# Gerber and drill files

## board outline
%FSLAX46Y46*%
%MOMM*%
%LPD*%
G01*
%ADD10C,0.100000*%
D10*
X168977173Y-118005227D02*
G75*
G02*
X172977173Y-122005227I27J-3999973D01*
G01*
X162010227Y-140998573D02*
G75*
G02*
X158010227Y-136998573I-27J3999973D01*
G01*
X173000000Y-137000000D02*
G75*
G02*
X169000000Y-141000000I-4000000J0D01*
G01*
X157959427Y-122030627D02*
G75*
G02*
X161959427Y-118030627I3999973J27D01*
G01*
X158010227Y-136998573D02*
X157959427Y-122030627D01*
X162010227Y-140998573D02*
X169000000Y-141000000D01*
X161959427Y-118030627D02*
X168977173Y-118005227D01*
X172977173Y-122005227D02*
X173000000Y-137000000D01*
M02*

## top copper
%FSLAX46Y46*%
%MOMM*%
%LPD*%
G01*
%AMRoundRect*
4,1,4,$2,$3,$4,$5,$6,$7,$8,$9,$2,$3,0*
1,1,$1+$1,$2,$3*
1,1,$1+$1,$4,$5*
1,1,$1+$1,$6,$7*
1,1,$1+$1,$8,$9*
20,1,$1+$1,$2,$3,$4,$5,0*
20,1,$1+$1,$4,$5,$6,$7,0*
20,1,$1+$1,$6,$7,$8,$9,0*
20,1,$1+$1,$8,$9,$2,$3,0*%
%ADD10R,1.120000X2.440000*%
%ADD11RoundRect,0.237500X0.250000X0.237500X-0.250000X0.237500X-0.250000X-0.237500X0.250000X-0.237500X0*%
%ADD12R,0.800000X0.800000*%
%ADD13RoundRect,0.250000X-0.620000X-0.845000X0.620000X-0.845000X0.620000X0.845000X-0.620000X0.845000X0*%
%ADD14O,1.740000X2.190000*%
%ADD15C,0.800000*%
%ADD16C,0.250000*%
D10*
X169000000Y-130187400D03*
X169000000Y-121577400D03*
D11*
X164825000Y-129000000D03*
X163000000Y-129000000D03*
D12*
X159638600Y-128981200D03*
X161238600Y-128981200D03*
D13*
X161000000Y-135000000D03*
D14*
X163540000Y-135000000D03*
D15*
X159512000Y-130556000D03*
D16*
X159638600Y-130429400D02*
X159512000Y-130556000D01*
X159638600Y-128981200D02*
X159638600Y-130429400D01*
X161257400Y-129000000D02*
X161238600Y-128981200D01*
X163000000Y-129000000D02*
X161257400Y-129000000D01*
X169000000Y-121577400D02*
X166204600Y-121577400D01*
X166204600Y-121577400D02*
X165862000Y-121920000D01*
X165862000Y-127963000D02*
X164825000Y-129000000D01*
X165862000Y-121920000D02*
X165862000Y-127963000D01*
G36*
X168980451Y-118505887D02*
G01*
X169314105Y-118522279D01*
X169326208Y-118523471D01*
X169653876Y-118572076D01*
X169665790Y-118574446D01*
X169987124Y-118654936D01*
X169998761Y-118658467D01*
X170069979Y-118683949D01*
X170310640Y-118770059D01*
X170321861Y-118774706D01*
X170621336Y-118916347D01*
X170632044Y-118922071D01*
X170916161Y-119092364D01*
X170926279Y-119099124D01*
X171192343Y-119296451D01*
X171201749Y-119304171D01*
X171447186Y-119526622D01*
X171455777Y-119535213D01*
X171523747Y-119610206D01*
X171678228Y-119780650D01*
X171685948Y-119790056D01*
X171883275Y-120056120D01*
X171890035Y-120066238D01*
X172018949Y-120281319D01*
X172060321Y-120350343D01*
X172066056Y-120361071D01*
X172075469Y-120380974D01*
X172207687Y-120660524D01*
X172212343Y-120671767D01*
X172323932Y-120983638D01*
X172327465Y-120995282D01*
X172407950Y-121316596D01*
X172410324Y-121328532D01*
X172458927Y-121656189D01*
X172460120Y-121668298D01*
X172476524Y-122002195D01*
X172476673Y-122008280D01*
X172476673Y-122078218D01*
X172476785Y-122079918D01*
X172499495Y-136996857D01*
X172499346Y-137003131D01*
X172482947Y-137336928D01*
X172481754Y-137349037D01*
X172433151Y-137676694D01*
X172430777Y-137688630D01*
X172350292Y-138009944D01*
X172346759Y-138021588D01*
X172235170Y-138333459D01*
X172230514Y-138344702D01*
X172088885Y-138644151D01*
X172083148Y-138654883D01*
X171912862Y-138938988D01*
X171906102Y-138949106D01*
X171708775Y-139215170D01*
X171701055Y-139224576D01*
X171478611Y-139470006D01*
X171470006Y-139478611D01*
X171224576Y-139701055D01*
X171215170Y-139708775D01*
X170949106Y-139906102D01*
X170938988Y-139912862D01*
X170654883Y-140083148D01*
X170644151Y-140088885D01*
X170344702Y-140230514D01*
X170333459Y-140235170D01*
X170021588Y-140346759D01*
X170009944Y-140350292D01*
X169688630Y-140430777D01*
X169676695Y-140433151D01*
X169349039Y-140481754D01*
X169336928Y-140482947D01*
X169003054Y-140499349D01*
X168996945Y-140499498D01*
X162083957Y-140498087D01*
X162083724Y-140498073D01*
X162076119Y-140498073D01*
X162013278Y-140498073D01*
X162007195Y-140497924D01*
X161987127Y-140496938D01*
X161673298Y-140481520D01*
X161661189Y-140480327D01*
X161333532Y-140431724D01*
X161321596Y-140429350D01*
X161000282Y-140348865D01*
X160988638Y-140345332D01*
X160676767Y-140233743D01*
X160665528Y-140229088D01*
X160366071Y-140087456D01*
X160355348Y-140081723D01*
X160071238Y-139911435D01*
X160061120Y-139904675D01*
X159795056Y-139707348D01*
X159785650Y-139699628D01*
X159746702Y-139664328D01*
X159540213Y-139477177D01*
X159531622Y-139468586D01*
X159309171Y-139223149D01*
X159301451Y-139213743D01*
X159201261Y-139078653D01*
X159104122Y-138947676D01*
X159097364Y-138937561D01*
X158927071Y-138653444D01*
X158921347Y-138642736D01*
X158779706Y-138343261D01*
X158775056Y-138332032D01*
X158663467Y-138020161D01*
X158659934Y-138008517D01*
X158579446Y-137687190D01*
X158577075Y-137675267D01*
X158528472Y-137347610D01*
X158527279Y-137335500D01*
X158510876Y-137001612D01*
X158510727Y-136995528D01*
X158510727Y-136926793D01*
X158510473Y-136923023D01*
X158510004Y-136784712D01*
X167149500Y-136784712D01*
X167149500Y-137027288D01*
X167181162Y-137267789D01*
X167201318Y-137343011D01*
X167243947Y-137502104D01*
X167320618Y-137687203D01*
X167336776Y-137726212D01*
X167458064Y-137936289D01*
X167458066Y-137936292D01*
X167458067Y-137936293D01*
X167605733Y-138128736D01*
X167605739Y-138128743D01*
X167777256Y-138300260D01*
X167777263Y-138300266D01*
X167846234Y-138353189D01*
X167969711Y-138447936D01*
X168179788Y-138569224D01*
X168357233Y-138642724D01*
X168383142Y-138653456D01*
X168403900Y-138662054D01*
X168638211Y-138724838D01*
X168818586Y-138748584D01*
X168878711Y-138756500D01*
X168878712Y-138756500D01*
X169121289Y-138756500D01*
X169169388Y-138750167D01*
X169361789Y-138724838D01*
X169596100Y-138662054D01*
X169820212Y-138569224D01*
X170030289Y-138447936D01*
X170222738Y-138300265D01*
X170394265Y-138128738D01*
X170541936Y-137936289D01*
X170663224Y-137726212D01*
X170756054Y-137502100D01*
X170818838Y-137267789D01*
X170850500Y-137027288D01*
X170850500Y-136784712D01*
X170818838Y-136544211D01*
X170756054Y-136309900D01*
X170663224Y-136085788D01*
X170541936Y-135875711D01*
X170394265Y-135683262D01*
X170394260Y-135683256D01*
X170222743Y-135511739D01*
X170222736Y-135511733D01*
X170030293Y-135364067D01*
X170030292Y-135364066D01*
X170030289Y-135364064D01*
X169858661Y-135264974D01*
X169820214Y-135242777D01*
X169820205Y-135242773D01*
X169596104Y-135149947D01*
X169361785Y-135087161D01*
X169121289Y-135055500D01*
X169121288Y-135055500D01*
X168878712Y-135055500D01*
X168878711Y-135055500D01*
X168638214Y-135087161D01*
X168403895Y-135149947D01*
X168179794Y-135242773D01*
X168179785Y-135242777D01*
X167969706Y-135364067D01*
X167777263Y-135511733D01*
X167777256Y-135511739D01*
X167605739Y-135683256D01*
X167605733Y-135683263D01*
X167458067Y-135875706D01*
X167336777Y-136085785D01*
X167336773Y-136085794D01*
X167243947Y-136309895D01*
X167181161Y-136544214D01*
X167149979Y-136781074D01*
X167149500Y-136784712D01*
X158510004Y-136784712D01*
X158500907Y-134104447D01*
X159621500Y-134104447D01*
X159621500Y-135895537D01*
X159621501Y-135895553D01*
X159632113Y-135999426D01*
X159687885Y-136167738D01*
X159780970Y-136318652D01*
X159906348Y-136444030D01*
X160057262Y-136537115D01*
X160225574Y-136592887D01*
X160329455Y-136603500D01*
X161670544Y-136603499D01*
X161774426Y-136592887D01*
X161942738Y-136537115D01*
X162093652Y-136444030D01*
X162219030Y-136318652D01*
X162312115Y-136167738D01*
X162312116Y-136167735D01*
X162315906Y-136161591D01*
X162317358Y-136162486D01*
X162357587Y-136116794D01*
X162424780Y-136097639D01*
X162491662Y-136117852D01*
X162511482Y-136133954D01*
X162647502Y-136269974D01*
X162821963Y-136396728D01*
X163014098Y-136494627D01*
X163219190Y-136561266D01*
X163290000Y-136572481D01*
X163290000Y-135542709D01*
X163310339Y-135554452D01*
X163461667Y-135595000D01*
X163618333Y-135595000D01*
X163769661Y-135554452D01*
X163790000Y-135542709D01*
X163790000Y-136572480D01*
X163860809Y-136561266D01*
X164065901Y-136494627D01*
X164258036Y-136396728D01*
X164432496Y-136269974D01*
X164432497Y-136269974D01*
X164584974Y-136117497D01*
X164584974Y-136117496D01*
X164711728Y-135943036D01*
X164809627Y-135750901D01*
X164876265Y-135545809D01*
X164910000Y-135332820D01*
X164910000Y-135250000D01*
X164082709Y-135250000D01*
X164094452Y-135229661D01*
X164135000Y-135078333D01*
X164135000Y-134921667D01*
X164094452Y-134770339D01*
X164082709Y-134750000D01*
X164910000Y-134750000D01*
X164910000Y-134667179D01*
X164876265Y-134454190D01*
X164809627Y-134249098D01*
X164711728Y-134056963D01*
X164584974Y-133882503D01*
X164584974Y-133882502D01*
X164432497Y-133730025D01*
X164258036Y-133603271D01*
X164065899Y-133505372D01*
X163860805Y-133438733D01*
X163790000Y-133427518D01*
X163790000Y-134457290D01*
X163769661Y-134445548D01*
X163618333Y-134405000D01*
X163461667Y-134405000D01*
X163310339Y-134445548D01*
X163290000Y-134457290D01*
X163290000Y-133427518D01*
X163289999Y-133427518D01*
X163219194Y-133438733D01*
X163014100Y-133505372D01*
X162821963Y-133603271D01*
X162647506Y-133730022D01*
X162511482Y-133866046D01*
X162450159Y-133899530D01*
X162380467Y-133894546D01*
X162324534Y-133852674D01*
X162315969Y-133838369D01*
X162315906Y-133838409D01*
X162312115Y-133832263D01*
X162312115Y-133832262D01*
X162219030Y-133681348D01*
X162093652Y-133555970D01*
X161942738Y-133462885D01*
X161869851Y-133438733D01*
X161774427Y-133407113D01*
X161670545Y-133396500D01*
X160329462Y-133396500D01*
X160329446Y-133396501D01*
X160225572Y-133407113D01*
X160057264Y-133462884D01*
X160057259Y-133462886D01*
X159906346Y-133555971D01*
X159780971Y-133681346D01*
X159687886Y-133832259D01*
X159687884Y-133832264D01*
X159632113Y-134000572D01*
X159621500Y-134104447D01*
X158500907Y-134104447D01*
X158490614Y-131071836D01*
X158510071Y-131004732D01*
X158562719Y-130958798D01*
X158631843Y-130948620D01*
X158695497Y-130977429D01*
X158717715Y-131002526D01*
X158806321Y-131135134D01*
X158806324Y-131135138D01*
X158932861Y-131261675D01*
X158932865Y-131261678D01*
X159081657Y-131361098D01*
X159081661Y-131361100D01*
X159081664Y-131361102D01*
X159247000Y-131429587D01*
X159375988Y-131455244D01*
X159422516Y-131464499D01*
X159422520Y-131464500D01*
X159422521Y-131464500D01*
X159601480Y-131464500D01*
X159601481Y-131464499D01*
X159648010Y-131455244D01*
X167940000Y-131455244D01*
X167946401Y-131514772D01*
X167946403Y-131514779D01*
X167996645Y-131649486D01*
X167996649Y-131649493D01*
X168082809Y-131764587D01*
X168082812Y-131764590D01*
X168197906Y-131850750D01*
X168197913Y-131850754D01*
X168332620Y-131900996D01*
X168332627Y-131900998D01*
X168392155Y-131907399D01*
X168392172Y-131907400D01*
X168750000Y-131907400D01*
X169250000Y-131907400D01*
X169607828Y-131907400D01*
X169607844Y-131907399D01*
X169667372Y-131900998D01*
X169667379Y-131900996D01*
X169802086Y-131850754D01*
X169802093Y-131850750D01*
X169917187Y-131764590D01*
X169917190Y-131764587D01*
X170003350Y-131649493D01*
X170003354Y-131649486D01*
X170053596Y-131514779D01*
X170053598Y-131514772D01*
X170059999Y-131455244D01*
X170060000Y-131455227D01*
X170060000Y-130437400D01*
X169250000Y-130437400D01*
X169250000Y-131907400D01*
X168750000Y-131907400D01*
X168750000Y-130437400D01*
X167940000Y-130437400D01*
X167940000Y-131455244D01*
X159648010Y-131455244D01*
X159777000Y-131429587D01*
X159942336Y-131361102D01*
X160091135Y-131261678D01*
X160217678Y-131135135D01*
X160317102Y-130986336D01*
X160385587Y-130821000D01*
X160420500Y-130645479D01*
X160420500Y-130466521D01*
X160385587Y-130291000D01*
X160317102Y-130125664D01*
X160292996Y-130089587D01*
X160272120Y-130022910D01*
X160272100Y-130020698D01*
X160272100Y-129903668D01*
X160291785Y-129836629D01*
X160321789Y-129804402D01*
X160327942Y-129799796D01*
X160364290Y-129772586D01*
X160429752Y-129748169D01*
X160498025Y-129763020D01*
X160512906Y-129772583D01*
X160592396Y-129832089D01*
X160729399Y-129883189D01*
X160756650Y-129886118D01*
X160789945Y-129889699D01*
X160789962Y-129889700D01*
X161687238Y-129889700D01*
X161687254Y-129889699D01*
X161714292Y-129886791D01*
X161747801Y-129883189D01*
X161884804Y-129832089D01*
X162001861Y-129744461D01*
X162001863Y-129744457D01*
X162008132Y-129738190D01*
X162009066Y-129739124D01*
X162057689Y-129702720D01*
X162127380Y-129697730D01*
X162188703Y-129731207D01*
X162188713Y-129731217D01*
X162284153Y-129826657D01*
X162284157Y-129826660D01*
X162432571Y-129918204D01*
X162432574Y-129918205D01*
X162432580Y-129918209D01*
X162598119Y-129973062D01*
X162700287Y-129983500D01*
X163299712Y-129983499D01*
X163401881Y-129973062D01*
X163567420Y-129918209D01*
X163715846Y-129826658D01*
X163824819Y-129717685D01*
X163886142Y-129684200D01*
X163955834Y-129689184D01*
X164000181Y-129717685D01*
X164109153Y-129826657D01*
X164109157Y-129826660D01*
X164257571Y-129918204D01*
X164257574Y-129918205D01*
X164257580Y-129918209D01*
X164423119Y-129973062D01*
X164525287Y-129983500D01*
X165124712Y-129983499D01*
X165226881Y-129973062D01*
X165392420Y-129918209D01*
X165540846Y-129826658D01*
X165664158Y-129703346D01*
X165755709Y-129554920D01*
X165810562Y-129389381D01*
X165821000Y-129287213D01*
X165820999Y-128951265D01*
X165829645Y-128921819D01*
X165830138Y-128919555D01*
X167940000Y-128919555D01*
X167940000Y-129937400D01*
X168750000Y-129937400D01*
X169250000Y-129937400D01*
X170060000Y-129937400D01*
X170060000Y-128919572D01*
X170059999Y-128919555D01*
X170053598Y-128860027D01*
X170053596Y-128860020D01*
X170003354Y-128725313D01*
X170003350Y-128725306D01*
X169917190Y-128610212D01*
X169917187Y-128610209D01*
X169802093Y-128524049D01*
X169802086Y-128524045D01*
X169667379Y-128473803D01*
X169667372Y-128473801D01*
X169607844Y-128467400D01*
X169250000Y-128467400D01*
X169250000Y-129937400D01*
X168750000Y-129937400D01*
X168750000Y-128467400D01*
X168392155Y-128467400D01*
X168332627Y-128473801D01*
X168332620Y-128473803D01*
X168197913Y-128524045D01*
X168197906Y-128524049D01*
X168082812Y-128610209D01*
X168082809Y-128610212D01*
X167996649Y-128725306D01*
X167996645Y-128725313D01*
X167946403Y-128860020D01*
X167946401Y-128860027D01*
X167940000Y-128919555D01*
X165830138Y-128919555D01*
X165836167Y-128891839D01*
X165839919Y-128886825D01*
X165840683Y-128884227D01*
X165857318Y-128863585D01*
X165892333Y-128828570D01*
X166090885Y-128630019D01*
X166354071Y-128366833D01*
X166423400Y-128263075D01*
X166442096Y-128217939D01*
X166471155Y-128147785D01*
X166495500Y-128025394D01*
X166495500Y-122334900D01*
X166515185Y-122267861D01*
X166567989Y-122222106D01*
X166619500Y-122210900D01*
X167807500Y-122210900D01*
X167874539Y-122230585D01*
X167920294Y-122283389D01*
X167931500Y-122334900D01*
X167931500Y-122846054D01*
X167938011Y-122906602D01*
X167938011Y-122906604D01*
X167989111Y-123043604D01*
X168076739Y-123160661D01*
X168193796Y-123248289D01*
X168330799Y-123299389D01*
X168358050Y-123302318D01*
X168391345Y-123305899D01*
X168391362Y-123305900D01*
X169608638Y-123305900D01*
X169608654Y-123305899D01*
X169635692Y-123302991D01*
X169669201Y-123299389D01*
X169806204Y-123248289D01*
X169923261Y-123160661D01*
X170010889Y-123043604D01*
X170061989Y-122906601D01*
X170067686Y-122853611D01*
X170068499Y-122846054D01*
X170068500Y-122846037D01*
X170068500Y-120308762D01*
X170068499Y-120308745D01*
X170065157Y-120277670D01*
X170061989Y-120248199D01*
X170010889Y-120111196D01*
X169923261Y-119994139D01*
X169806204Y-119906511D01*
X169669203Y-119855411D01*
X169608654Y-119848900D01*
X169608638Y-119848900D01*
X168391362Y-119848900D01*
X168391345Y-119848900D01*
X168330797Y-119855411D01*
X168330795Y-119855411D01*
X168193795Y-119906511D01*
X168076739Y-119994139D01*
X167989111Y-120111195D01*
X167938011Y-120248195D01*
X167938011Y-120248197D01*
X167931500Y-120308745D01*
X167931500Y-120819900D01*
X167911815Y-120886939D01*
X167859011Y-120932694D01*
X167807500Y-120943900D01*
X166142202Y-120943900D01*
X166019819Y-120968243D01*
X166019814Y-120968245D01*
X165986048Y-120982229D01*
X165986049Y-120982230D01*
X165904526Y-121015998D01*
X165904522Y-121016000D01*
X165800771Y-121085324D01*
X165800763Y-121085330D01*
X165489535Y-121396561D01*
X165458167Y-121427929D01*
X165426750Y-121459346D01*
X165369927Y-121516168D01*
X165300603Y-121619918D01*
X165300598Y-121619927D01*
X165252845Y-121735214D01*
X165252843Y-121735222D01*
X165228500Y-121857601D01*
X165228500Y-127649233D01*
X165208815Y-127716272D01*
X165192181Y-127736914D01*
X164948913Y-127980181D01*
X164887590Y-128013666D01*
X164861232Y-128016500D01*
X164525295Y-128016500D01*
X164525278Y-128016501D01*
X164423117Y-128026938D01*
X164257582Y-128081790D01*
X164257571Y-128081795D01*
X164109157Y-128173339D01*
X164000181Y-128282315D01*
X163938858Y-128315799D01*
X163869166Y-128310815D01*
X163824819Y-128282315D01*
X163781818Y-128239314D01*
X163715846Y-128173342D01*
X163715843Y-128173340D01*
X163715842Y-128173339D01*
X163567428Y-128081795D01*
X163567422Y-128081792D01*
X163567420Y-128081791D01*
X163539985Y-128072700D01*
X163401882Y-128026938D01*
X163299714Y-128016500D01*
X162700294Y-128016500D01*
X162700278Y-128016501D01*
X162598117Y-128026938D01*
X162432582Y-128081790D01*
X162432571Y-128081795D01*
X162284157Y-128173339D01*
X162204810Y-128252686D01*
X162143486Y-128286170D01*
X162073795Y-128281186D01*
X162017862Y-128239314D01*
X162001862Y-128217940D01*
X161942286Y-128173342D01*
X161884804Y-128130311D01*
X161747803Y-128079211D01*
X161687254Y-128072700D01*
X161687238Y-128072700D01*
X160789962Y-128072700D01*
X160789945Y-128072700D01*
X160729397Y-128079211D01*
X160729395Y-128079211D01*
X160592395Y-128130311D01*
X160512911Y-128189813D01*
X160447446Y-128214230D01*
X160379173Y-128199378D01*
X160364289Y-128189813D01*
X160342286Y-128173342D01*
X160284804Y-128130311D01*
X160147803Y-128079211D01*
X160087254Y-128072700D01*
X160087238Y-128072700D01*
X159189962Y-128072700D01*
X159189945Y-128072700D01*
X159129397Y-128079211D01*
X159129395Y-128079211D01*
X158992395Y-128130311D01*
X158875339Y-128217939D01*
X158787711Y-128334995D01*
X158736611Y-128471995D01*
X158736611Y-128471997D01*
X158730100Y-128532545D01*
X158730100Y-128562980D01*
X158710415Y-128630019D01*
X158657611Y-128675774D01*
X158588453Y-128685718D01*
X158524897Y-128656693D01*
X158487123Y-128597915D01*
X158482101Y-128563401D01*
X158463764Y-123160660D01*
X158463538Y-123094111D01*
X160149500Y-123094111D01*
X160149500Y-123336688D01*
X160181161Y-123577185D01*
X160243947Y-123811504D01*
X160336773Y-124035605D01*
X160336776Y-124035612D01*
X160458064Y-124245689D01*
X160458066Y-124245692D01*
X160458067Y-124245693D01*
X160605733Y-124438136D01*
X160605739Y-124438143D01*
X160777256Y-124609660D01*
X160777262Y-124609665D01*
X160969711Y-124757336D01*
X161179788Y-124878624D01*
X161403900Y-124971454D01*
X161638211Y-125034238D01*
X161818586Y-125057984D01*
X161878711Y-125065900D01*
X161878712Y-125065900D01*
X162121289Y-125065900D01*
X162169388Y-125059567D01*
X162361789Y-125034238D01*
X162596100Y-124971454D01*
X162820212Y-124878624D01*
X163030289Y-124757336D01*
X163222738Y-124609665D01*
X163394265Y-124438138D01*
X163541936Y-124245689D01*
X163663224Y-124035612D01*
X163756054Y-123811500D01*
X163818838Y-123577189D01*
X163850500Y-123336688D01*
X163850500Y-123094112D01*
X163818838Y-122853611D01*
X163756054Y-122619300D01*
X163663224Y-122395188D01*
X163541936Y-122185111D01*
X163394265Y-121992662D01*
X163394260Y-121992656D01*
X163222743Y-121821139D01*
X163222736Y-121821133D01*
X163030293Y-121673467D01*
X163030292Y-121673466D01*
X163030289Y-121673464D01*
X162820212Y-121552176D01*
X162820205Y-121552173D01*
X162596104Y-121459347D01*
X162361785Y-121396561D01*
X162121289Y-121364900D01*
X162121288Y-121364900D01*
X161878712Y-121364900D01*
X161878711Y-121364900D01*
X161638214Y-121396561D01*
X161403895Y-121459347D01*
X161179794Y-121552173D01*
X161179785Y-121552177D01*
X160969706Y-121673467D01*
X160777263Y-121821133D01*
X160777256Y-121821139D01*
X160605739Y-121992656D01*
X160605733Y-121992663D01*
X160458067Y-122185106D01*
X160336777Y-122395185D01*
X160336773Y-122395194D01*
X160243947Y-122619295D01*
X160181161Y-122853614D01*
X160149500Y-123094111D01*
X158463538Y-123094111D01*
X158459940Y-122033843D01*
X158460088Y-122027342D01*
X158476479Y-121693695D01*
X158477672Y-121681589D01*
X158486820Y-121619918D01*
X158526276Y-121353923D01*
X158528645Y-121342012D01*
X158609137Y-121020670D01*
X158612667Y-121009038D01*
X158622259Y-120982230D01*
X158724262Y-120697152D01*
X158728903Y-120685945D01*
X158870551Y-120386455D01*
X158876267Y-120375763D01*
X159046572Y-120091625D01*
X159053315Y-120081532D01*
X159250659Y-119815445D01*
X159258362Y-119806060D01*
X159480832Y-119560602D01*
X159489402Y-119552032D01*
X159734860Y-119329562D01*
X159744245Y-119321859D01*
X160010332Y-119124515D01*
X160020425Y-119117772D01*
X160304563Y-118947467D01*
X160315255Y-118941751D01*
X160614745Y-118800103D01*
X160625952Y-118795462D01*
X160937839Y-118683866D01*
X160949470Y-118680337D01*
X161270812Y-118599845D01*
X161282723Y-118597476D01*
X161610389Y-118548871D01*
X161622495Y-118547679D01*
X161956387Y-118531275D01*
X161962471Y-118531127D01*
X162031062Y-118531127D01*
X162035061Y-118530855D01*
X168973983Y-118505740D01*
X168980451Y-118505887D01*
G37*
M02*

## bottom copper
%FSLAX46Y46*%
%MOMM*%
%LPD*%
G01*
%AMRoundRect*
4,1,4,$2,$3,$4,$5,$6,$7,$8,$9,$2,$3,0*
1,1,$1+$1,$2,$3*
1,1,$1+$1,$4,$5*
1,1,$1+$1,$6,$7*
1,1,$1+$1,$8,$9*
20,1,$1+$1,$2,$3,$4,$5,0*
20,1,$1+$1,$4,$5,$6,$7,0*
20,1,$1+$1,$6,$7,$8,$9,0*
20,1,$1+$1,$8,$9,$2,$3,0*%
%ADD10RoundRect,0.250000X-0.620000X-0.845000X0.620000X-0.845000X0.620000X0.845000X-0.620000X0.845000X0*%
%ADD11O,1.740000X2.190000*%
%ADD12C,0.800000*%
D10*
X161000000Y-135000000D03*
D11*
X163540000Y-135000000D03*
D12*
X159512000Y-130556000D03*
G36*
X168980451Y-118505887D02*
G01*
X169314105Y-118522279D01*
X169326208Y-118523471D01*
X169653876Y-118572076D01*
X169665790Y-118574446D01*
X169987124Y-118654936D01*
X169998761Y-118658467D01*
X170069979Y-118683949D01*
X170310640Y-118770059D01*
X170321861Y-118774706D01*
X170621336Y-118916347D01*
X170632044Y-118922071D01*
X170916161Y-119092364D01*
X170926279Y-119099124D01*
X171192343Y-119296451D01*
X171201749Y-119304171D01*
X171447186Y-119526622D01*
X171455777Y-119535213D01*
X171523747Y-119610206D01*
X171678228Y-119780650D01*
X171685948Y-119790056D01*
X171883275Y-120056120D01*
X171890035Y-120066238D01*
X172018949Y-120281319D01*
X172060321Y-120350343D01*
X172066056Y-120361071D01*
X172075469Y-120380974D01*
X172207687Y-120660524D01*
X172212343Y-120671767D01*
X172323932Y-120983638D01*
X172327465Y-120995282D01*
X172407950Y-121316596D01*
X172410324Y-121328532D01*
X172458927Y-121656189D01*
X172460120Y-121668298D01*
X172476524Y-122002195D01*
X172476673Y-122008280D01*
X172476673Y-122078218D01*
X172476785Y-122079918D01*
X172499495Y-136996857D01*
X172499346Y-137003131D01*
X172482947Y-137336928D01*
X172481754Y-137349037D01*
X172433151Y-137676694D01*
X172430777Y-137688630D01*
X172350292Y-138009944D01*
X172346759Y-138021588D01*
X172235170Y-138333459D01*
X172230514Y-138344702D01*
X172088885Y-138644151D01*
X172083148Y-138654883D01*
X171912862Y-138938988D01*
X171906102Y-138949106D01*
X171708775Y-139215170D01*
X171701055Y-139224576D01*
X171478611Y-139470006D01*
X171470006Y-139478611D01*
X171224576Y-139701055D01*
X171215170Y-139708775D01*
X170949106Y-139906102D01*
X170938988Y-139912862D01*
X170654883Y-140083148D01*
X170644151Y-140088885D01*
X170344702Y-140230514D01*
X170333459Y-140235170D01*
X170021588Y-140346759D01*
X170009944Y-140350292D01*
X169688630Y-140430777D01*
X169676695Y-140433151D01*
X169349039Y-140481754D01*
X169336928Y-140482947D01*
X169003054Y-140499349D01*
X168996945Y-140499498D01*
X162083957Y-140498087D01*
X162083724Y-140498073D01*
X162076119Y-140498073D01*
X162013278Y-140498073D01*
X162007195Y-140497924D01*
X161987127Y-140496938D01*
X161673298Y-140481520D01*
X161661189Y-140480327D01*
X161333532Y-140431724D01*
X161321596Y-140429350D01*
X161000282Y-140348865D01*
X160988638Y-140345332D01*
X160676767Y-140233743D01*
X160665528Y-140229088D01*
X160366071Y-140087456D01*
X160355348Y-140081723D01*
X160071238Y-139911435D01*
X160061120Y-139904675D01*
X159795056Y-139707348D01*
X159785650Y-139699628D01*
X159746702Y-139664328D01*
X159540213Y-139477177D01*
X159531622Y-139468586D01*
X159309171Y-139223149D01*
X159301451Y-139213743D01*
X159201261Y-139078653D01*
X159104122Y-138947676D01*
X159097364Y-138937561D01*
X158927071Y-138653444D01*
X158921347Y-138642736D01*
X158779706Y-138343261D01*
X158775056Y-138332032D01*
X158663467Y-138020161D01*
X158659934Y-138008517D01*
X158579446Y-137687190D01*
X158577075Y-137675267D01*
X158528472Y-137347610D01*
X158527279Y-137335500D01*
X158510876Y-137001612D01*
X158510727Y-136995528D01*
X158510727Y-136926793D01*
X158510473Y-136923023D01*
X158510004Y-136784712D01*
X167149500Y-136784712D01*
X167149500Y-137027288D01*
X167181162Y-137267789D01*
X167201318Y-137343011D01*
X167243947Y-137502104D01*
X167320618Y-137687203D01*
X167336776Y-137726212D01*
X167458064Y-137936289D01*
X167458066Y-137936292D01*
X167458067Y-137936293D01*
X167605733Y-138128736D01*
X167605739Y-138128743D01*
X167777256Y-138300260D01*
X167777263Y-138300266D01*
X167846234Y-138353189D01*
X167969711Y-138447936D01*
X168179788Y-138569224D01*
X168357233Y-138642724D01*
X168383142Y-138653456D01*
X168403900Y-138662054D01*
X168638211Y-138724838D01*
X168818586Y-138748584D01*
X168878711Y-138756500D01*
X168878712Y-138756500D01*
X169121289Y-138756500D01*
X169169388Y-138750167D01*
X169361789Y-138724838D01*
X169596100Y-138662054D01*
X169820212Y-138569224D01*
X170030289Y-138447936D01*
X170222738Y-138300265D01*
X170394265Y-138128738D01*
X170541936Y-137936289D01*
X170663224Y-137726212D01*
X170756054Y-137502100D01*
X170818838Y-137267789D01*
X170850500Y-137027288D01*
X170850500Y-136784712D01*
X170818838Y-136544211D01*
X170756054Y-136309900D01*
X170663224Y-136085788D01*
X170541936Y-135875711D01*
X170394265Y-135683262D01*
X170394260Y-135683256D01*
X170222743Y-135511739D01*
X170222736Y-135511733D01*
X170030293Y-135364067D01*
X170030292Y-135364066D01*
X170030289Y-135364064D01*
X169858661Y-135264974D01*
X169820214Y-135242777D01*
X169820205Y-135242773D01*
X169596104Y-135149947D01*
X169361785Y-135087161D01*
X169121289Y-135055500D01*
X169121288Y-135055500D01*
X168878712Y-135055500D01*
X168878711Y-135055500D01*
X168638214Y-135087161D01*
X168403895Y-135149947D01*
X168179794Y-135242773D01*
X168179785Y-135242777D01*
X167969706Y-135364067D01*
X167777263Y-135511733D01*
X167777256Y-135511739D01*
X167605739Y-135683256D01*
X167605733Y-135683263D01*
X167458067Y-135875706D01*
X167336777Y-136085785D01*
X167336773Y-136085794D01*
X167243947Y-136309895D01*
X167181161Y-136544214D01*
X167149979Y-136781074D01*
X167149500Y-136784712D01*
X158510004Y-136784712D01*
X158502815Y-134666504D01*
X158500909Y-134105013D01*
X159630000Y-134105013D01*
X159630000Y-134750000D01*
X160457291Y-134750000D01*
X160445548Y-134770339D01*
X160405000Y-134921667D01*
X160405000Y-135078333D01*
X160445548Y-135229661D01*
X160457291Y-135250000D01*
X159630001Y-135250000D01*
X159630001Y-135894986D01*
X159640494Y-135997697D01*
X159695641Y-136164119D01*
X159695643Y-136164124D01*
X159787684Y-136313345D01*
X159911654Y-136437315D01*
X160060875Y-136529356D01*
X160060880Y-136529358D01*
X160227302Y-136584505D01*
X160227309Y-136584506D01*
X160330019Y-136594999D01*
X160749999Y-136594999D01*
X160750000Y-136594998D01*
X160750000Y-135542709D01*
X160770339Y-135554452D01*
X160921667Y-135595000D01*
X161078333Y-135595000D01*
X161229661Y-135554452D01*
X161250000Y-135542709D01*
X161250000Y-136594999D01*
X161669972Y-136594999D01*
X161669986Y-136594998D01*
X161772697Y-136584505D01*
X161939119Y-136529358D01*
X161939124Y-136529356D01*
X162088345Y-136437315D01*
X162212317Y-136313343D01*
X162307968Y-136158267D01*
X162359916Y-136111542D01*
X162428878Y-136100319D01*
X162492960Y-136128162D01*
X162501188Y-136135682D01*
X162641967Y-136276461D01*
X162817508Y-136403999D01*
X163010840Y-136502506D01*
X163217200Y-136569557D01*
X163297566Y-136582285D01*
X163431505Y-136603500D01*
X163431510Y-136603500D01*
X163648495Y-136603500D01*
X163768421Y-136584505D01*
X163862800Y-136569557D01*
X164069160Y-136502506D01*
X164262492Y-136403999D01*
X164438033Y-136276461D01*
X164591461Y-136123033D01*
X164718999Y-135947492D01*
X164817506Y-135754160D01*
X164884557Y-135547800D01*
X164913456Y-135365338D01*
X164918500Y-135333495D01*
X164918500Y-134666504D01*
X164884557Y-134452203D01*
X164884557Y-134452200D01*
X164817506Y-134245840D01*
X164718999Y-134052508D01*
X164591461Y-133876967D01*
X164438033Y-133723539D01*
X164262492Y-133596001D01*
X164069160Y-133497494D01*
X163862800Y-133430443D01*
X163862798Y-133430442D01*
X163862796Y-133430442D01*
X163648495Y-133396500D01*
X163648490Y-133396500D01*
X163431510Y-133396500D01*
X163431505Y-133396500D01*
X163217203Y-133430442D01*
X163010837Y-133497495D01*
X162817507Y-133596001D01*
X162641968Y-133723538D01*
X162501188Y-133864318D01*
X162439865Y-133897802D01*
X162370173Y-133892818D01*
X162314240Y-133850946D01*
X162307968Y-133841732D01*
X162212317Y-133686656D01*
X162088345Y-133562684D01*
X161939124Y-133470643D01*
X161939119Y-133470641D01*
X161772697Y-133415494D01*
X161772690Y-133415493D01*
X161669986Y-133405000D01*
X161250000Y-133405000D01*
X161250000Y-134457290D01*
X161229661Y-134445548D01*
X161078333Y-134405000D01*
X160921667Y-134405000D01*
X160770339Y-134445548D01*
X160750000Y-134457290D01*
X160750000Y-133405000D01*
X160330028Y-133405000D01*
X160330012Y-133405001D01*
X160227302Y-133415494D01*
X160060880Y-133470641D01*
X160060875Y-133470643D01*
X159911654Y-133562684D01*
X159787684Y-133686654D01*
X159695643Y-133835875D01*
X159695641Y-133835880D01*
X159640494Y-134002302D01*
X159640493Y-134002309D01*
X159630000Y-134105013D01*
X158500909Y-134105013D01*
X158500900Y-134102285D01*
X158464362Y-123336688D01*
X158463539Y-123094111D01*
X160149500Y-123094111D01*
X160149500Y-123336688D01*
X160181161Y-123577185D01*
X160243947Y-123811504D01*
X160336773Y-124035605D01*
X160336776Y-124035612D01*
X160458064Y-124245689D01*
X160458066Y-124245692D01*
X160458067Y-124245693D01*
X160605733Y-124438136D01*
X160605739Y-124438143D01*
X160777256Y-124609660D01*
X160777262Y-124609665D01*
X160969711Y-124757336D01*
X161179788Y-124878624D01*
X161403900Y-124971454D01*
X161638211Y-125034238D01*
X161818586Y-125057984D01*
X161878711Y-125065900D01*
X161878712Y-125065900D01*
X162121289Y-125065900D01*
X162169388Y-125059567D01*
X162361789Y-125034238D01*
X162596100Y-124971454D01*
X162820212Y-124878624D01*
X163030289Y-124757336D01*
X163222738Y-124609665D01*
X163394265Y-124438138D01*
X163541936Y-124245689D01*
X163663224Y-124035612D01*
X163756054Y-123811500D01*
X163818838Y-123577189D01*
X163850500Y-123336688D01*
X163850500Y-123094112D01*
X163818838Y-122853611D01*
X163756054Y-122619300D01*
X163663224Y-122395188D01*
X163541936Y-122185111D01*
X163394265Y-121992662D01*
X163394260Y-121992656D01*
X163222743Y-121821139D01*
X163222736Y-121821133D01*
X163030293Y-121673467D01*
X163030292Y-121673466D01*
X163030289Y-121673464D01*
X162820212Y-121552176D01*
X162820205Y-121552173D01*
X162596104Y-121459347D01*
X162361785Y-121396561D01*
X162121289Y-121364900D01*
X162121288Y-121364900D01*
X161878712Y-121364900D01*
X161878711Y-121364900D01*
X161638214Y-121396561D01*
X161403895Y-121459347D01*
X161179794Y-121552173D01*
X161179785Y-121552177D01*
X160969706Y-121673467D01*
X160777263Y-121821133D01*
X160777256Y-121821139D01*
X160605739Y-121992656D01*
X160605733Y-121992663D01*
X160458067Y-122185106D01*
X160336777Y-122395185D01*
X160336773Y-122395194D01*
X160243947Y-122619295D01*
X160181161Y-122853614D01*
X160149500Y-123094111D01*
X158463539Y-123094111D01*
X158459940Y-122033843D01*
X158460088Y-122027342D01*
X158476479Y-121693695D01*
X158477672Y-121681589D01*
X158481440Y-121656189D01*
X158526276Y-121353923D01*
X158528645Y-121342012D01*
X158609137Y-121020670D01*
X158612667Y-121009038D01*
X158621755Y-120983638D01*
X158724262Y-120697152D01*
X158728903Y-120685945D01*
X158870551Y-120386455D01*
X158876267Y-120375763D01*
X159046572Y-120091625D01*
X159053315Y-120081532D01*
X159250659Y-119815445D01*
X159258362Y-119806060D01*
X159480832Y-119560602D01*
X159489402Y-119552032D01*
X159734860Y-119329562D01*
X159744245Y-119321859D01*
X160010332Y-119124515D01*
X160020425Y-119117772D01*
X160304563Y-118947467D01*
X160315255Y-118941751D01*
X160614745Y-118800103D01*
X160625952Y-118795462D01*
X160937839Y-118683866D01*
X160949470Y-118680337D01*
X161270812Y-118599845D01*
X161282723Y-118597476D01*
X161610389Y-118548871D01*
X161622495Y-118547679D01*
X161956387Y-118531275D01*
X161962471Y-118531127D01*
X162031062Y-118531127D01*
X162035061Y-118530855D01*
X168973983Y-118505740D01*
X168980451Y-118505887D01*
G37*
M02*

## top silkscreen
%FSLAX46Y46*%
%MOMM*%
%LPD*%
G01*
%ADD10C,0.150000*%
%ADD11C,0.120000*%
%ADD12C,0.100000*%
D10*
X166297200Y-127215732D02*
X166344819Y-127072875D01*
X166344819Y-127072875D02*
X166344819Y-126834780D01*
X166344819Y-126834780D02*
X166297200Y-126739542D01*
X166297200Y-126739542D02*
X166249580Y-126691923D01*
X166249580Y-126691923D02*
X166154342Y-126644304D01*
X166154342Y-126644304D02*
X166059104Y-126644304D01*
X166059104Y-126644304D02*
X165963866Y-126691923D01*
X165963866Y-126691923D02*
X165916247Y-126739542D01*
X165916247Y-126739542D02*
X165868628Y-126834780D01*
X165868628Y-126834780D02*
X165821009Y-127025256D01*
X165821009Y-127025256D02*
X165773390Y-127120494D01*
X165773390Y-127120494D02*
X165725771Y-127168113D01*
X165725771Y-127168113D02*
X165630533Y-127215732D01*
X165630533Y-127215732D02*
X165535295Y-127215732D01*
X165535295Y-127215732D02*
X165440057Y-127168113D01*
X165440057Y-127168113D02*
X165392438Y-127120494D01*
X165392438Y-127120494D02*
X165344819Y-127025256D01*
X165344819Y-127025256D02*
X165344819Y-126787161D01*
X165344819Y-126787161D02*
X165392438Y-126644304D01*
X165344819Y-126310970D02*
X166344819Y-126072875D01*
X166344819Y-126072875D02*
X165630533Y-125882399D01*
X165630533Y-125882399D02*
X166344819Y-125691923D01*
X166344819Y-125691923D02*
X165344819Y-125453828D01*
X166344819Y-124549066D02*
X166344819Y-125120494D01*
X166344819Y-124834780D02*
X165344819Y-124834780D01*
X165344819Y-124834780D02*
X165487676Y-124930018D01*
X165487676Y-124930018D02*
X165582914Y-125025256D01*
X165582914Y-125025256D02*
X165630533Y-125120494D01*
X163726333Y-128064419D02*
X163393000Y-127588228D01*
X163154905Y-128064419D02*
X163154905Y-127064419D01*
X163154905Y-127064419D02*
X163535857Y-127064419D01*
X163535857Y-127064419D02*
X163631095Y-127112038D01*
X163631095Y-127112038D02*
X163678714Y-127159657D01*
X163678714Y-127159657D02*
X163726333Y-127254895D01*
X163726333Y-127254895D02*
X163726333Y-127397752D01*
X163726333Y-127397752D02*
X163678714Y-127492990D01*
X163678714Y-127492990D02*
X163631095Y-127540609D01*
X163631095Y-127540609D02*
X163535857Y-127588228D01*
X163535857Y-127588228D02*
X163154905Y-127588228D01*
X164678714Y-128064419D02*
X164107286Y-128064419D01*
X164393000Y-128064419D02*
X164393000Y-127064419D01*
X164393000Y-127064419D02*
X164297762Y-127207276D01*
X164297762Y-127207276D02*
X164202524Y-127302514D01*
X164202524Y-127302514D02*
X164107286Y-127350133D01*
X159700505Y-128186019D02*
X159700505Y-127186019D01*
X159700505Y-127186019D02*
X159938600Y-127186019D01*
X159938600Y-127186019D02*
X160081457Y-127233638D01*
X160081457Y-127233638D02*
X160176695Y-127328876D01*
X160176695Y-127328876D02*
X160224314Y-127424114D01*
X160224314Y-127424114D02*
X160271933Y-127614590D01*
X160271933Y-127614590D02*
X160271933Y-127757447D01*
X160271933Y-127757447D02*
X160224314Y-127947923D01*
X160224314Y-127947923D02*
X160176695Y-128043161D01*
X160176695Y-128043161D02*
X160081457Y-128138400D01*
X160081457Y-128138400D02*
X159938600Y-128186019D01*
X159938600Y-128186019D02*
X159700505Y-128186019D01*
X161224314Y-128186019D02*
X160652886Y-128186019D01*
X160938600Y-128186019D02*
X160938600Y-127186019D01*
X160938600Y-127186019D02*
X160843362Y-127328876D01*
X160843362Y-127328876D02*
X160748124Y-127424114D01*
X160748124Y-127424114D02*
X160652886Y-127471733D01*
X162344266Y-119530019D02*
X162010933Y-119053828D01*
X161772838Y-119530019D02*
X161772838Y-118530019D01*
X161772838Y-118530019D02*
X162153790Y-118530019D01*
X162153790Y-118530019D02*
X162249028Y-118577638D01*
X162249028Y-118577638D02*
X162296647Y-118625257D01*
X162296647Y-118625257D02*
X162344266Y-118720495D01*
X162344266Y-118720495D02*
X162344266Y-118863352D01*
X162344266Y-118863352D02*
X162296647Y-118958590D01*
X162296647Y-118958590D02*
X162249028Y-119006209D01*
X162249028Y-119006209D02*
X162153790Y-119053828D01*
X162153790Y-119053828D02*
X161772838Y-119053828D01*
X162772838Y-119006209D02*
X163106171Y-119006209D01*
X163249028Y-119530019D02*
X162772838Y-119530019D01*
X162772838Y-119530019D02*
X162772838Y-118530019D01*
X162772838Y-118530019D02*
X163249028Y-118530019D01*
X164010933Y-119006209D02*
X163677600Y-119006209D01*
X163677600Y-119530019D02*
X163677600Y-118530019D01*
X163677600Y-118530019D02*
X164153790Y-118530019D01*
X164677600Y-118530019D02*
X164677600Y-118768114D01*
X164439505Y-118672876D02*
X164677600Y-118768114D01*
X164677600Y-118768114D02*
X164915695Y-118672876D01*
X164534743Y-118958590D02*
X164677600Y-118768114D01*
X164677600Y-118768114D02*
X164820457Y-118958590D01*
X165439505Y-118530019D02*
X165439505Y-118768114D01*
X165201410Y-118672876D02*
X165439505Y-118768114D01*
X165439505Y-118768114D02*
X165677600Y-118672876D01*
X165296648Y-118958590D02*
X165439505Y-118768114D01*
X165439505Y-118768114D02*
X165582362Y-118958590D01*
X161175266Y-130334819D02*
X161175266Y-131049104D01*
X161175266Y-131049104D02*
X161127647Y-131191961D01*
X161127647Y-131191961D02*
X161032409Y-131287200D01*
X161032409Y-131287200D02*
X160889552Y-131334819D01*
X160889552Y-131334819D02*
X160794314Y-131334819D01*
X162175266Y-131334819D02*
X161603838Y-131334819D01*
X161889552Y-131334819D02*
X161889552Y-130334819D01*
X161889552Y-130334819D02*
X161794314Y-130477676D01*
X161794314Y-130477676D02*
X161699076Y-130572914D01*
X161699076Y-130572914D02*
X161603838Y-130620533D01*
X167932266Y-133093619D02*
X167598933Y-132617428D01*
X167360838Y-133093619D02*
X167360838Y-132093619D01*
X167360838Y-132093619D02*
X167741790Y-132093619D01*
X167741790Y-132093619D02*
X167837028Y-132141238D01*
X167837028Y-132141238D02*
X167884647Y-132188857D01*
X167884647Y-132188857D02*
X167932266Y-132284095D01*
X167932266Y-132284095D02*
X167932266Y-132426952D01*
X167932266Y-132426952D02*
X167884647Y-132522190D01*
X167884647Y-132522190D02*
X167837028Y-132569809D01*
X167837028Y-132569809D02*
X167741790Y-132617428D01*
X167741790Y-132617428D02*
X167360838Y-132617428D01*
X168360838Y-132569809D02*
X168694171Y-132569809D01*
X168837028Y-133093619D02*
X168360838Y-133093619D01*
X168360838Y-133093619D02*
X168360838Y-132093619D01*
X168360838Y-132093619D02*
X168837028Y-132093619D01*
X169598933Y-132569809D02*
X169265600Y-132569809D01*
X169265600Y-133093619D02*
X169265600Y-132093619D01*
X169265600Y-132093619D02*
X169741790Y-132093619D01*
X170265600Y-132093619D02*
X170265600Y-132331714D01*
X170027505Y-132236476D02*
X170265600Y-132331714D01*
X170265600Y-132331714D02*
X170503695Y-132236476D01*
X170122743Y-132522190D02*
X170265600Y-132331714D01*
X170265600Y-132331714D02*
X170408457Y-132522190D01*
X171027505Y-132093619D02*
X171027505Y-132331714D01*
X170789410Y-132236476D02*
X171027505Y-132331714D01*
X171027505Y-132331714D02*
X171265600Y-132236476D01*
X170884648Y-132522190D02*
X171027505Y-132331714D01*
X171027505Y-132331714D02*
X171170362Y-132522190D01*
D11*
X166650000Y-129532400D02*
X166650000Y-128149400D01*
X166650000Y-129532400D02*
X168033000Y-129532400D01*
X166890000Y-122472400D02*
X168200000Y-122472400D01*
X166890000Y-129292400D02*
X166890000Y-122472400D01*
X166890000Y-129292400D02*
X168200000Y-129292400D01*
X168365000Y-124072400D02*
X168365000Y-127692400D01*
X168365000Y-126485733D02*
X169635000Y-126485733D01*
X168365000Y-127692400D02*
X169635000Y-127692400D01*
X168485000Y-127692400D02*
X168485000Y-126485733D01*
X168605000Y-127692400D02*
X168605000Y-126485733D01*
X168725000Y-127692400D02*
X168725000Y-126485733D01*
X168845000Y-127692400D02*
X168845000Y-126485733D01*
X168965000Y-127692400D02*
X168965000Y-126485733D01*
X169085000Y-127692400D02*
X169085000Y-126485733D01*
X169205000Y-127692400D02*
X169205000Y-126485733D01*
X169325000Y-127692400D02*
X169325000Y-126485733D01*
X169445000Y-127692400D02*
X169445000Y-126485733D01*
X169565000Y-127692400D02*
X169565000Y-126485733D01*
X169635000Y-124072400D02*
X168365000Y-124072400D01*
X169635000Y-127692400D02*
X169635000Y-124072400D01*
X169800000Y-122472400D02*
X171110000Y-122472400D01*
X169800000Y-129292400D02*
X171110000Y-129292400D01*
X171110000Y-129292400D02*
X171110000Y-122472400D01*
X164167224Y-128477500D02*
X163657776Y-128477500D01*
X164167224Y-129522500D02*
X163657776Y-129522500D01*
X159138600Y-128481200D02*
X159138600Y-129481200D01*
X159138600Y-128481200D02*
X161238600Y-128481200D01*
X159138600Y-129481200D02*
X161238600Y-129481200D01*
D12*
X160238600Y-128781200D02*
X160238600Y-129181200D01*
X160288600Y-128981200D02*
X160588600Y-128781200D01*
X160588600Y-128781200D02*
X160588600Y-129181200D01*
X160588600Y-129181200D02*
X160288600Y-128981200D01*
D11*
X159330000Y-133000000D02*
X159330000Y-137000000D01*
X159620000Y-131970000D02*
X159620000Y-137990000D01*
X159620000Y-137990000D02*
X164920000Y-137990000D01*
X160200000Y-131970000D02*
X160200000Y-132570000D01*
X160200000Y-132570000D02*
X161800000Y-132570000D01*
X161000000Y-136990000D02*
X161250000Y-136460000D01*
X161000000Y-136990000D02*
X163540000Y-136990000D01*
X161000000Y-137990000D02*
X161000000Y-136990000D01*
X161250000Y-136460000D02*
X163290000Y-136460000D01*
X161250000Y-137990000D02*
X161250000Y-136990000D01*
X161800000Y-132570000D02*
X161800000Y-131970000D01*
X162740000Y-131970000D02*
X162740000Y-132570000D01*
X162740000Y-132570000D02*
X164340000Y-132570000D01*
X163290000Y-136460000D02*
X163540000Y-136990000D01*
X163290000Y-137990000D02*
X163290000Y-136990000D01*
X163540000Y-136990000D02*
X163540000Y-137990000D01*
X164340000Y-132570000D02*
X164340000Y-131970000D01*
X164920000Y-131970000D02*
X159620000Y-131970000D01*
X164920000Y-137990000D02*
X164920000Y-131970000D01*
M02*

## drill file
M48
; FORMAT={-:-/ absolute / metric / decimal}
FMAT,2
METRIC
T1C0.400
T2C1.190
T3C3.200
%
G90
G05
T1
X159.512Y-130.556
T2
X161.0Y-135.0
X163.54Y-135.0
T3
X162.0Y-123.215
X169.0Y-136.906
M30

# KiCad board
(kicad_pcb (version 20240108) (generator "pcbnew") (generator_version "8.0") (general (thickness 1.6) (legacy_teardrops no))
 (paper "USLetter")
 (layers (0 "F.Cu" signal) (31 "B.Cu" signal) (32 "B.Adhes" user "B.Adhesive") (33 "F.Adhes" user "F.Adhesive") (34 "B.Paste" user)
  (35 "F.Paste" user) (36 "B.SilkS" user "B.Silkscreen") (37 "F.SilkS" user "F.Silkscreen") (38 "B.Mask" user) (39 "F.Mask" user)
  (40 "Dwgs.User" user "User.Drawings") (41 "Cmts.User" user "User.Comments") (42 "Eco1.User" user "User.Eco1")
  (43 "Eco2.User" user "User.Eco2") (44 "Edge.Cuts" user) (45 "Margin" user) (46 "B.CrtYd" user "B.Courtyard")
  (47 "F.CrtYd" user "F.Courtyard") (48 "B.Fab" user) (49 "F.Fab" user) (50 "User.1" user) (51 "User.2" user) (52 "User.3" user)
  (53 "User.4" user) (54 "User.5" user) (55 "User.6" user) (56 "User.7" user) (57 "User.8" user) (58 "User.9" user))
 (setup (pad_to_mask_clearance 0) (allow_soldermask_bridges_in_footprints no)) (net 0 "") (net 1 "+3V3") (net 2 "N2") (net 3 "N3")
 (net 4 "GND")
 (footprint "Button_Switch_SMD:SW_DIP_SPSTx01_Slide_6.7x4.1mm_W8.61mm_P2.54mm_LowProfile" (layer "F.Cu") (at 169 125.8824 90)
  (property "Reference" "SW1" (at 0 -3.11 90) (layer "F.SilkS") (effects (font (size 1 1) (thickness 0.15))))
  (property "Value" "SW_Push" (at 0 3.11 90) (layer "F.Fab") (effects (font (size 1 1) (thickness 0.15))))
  (fp_line (start -3.65 -2.35) (end -2.267 -2.35) (stroke (width 0.12) (type solid)) (layer "F.SilkS"))
  (fp_line (start -3.65 -2.35) (end -3.65 -0.967) (stroke (width 0.12) (type solid)) (layer "F.SilkS"))
  (fp_line (start 3.41 -2.11) (end 3.41 -0.8) (stroke (width 0.12) (type solid)) (layer "F.SilkS"))
  (fp_line (start -3.41 -2.11) (end 3.41 -2.11) (stroke (width 0.12) (type solid)) (layer "F.SilkS"))
  (fp_line (start -3.41 -2.11) (end -3.41 -0.8) (stroke (width 0.12) (type solid)) (layer "F.SilkS"))
  (fp_line (start 1.81 -0.635) (end -1.81 -0.635) (stroke (width 0.12) (type solid)) (layer "F.SilkS"))
  (fp_line (start -0.603333 -0.635) (end -0.603333 0.635) (stroke (width 0.12) (type solid)) (layer "F.SilkS"))
  (fp_line (start -1.81 -0.635) (end -1.81 0.635) (stroke (width 0.12) (type solid)) (layer "F.SilkS"))
  (fp_line (start -1.81 -0.515) (end -0.603333 -0.515) (stroke (width 0.12) (type solid)) (layer "F.SilkS"))
  (fp_line (start -1.81 -0.395) (end -0.603333 -0.395) (stroke (width 0.12) (type solid)) (layer "F.SilkS"))
  (fp_line (start -1.81 -0.275) (end -0.603333 -0.275) (stroke (width 0.12) (type solid)) (layer "F.SilkS"))
  (fp_line (start -1.81 -0.155) (end -0.603333 -0.155) (stroke (width 0.12) (type solid)) (layer "F.SilkS"))
  (fp_line (start -1.81 -0.035) (end -0.603333 -0.035) (stroke (width 0.12) (type solid)) (layer "F.SilkS"))
  (fp_line (start -1.81 0.085) (end -0.603333 0.085) (stroke (width 0.12) (type solid)) (layer "F.SilkS"))
  (fp_line (start -1.81 0.205) (end -0.603333 0.205) (stroke (width 0.12) (type solid)) (layer "F.SilkS"))
  (fp_line (start -1.81 0.325) (end -0.603333 0.325) (stroke (width 0.12) (type solid)) (layer "F.SilkS"))
  (fp_line (start -1.81 0.445) (end -0.603333 0.445) (stroke (width 0.12) (type solid)) (layer "F.SilkS"))
  (fp_line (start -1.81 0.565) (end -0.603333 0.565) (stroke (width 0.12) (type solid)) (layer "F.SilkS"))
  (fp_line (start 1.81 0.635) (end 1.81 -0.635) (stroke (width 0.12) (type solid)) (layer "F.SilkS"))
  (fp_line (start -1.81 0.635) (end 1.81 0.635) (stroke (width 0.12) (type solid)) (layer "F.SilkS"))
  (fp_line (start 3.41 0.8) (end 3.41 2.11) (stroke (width 0.12) (type solid)) (layer "F.SilkS"))
  (fp_line (start -3.41 0.8) (end -3.41 2.11) (stroke (width 0.12) (type solid)) (layer "F.SilkS"))
  (fp_line (start -3.41 2.11) (end 3.41 2.11) (stroke (width 0.12) (type solid)) (layer "F.SilkS"))
  (pad "1" smd rect (at -4.305 0 90) (size 2.44 1.12) (layers "F.Cu" "F.Paste" "F.Mask") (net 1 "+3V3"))
  (pad "2" smd rect (at 4.305 0 90) (size 2.44 1.12) (layers "F.Cu" "F.Paste" "F.Mask") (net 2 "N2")))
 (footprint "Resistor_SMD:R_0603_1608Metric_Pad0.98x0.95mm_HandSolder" (layer "F.Cu") (at 163.9125 129 180)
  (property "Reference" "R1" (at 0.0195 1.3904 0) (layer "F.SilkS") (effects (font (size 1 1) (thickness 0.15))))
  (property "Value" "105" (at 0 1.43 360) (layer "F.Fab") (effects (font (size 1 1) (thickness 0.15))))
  (fp_line (start -0.254724 0.5225) (end 0.254724 0.5225) (stroke (width 0.12) (type solid)) (layer "F.SilkS"))
  (fp_line (start -0.254724 -0.5225) (end 0.254724 -0.5225) (stroke (width 0.12) (type solid)) (layer "F.SilkS"))
  (pad "1" smd roundrect (at -0.9125 0 180) (size 0.975 0.95) (layers "F.Cu" "F.Paste" "F.Mask") (roundrect_rratio 0.25) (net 2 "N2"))
  (pad "2" smd roundrect (at 0.9125 0 180) (size 0.975 0.95) (layers "F.Cu" "F.Paste" "F.Mask") (roundrect_rratio 0.25) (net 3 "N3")))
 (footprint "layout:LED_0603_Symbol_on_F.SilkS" (layer "F.Cu") (at 160.4386 128.9812)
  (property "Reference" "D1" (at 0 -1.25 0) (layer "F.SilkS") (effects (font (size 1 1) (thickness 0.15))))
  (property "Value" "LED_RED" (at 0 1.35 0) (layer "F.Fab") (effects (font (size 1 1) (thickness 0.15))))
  (fp_line (start -1.3 -0.5) (end -1.3 0.5) (stroke (width 0.12) (type solid)) (layer "F.SilkS"))
  (fp_line (start -1.3 -0.5) (end 0.8 -0.5) (stroke (width 0.12) (type solid)) (layer "F.SilkS"))
  (fp_line (start -1.3 0.5) (end 0.8 0.5) (stroke (width 0.12) (type solid)) (layer "F.SilkS"))
  (fp_line (start -0.2 -0.2) (end -0.2 0.2) (stroke (width 0.1) (type solid)) (layer "F.SilkS"))
  (fp_line (start -0.15 0) (end 0.15 -0.2) (stroke (width 0.1) (type solid)) (layer "F.SilkS"))
  (fp_line (start 0.15 -0.2) (end 0.15 0.2) (stroke (width 0.1) (type solid)) (layer "F.SilkS"))
  (fp_line (start 0.15 0.2) (end -0.15 0) (stroke (width 0.1) (type solid)) (layer "F.SilkS"))
  (pad "1" smd rect (at -0.8 0 180) (size 0.8 0.8) (layers "F.Cu" "F.Paste" "F.Mask") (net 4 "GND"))
  (pad "2" smd rect (at 0.8 0 180) (size 0.8 0.8) (layers "F.Cu" "F.Paste" "F.Mask") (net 3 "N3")))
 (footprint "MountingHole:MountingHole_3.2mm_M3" (layer "F.Cu") (at 169 136.906)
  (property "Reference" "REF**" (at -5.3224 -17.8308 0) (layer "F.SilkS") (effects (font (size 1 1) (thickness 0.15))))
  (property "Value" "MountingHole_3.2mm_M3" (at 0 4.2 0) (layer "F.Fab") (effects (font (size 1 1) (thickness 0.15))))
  (pad "" np_thru_hole circle (at 0 0) (size 3.2 3.2) (drill 3.2) (layers "*.Cu" "*.Mask")))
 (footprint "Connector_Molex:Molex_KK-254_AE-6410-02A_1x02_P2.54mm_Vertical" (layer "F.Cu") (at 161 135)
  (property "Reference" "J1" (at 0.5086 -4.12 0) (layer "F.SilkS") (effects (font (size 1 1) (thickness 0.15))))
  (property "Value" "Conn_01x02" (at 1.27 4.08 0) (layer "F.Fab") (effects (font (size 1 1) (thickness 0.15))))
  (fp_line (start -1.67 -2) (end -1.67 2) (stroke (width 0.12) (type solid)) (layer "F.SilkS"))
  (fp_line (start -1.38 -3.03) (end -1.38 2.99) (stroke (width 0.12) (type solid)) (layer "F.SilkS"))
  (fp_line (start -1.38 2.99) (end 3.92 2.99) (stroke (width 0.12) (type solid)) (layer "F.SilkS"))
  (fp_line (start -0.8 -3.03) (end -0.8 -2.43) (stroke (width 0.12) (type solid)) (layer "F.SilkS"))
  (fp_line (start -0.8 -2.43) (end 0.8 -2.43) (stroke (width 0.12) (type solid)) (layer "F.SilkS"))
  (fp_line (start 0 1.99) (end 0.25 1.46) (stroke (width 0.12) (type solid)) (layer "F.SilkS"))
  (fp_line (start 0 1.99) (end 2.54 1.99) (stroke (width 0.12) (type solid)) (layer "F.SilkS"))
  (fp_line (start 0 2.99) (end 0 1.99) (stroke (width 0.12) (type solid)) (layer "F.SilkS"))
  (fp_line (start 0.25 1.46) (end 2.29 1.46) (stroke (width 0.12) (type solid)) (layer "F.SilkS"))
  (fp_line (start 0.25 2.99) (end 0.25 1.99) (stroke (width 0.12) (type solid)) (layer "F.SilkS"))
  (fp_line (start 0.8 -2.43) (end 0.8 -3.03) (stroke (width 0.12) (type solid)) (layer "F.SilkS"))
  (fp_line (start 1.74 -3.03) (end 1.74 -2.43) (stroke (width 0.12) (type solid)) (layer "F.SilkS"))
  (fp_line (start 1.74 -2.43) (end 3.34 -2.43) (stroke (width 0.12) (type solid)) (layer "F.SilkS"))
  (fp_line (start 2.29 1.46) (end 2.54 1.99) (stroke (width 0.12) (type solid)) (layer "F.SilkS"))
  (fp_line (start 2.29 2.99) (end 2.29 1.99) (stroke (width 0.12) (type solid)) (layer "F.SilkS"))
  (fp_line (start 2.54 1.99) (end 2.54 2.99) (stroke (width 0.12) (type solid)) (layer "F.SilkS"))
  (fp_line (start 3.34 -2.43) (end 3.34 -3.03) (stroke (width 0.12) (type solid)) (layer "F.SilkS"))
  (fp_line (start 3.92 -3.03) (end -1.38 -3.03) (stroke (width 0.12) (type solid)) (layer "F.SilkS"))
  (fp_line (start 3.92 2.99) (end 3.92 -3.03) (stroke (width 0.12) (type solid)) (layer "F.SilkS"))
  (pad "1" thru_hole roundrect (at 0 0) (size 1.74 2.19) (drill 1.19) (layers "*.Cu" "*.Mask") (remove_unused_layers no)
   (roundrect_rratio 0.143678) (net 4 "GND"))
  (pad "2" thru_hole oval (at 2.54 0) (size 1.74 2.19) (drill 1.19) (layers "*.Cu" "*.Mask") (remove_unused_layers no) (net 1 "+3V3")))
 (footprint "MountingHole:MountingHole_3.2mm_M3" (layer "F.Cu") (at 162 123.2154)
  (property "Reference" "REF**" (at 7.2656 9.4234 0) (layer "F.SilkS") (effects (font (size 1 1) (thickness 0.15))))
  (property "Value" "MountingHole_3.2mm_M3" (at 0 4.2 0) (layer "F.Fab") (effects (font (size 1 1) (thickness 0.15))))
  (pad "" np_thru_hole circle (at 0 0) (size 3.2 3.2) (drill 3.2) (layers "*.Cu" "*.Mask")))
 (gr_arc (start 168.977173 118.005227) (mid 171.8056 119.1768) (end 172.977173 122.005227) (stroke (width 0.1) (type default))
  (layer "Edge.Cuts"))
 (gr_arc (start 162.010227 140.998573) (mid 159.1818 139.827) (end 158.010227 136.998573) (stroke (width 0.1) (type default))
  (layer "Edge.Cuts"))
 (gr_arc (start 173 137) (mid 171.828427 139.828427) (end 169 141) (stroke (width 0.1) (type default)) (layer "Edge.Cuts"))
 (gr_arc (start 157.959427 122.030627) (mid 159.131 119.2022) (end 161.959427 118.030627) (stroke (width 0.1) (type default))
  (layer "Edge.Cuts"))
 (gr_line (start 158.010227 136.998573) (end 157.959427 122.030627) (stroke (width 0.1) (type default)) (layer "Edge.Cuts"))
 (gr_line (start 162.010227 140.998573) (end 169 141) (stroke (width 0.1) (type default)) (layer "Edge.Cuts"))
 (gr_line (start 161.959427 118.030627) (end 168.977173 118.005227) (stroke (width 0.1) (type default)) (layer "Edge.Cuts"))
 (gr_line (start 172.977173 122.005227) (end 173 137) (stroke (width 0.1) (type default)) (layer "Edge.Cuts"))
 (segment (start 159.6386 130.4294) (end 159.512 130.556) (width 0.25) (layer "F.Cu") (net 4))
 (segment (start 159.6386 128.9812) (end 159.6386 130.4294) (width 0.25) (layer "F.Cu") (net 4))
 (via (at 159.512 130.556) (size 0.8) (drill 0.4) (layers "F.Cu" "B.Cu") (free yes) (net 4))
 (segment (start 161.2574 129) (end 161.2386 128.9812) (width 0.25) (layer "F.Cu") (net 3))
 (segment (start 163 129) (end 161.2574 129) (width 0.25) (layer "F.Cu") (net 3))
 (segment (start 169 121.5774) (end 166.2046 121.5774) (width 0.25) (layer "F.Cu") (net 2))
 (segment (start 166.2046 121.5774) (end 165.862 121.92) (width 0.25) (layer "F.Cu") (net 2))
 (segment (start 165.862 127.963) (end 164.825 129) (width 0.25) (layer "F.Cu") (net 2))
 (segment (start 165.862 121.92) (end 165.862 127.963) (width 0.25) (layer "F.Cu") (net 2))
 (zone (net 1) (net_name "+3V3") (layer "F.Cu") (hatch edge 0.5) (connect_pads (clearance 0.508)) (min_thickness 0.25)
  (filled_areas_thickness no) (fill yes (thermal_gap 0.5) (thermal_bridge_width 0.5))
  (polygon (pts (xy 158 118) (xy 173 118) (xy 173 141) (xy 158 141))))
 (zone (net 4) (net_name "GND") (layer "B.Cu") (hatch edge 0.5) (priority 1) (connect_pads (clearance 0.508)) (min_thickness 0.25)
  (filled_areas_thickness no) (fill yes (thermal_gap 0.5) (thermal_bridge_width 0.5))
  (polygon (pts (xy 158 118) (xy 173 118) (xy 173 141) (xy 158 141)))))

